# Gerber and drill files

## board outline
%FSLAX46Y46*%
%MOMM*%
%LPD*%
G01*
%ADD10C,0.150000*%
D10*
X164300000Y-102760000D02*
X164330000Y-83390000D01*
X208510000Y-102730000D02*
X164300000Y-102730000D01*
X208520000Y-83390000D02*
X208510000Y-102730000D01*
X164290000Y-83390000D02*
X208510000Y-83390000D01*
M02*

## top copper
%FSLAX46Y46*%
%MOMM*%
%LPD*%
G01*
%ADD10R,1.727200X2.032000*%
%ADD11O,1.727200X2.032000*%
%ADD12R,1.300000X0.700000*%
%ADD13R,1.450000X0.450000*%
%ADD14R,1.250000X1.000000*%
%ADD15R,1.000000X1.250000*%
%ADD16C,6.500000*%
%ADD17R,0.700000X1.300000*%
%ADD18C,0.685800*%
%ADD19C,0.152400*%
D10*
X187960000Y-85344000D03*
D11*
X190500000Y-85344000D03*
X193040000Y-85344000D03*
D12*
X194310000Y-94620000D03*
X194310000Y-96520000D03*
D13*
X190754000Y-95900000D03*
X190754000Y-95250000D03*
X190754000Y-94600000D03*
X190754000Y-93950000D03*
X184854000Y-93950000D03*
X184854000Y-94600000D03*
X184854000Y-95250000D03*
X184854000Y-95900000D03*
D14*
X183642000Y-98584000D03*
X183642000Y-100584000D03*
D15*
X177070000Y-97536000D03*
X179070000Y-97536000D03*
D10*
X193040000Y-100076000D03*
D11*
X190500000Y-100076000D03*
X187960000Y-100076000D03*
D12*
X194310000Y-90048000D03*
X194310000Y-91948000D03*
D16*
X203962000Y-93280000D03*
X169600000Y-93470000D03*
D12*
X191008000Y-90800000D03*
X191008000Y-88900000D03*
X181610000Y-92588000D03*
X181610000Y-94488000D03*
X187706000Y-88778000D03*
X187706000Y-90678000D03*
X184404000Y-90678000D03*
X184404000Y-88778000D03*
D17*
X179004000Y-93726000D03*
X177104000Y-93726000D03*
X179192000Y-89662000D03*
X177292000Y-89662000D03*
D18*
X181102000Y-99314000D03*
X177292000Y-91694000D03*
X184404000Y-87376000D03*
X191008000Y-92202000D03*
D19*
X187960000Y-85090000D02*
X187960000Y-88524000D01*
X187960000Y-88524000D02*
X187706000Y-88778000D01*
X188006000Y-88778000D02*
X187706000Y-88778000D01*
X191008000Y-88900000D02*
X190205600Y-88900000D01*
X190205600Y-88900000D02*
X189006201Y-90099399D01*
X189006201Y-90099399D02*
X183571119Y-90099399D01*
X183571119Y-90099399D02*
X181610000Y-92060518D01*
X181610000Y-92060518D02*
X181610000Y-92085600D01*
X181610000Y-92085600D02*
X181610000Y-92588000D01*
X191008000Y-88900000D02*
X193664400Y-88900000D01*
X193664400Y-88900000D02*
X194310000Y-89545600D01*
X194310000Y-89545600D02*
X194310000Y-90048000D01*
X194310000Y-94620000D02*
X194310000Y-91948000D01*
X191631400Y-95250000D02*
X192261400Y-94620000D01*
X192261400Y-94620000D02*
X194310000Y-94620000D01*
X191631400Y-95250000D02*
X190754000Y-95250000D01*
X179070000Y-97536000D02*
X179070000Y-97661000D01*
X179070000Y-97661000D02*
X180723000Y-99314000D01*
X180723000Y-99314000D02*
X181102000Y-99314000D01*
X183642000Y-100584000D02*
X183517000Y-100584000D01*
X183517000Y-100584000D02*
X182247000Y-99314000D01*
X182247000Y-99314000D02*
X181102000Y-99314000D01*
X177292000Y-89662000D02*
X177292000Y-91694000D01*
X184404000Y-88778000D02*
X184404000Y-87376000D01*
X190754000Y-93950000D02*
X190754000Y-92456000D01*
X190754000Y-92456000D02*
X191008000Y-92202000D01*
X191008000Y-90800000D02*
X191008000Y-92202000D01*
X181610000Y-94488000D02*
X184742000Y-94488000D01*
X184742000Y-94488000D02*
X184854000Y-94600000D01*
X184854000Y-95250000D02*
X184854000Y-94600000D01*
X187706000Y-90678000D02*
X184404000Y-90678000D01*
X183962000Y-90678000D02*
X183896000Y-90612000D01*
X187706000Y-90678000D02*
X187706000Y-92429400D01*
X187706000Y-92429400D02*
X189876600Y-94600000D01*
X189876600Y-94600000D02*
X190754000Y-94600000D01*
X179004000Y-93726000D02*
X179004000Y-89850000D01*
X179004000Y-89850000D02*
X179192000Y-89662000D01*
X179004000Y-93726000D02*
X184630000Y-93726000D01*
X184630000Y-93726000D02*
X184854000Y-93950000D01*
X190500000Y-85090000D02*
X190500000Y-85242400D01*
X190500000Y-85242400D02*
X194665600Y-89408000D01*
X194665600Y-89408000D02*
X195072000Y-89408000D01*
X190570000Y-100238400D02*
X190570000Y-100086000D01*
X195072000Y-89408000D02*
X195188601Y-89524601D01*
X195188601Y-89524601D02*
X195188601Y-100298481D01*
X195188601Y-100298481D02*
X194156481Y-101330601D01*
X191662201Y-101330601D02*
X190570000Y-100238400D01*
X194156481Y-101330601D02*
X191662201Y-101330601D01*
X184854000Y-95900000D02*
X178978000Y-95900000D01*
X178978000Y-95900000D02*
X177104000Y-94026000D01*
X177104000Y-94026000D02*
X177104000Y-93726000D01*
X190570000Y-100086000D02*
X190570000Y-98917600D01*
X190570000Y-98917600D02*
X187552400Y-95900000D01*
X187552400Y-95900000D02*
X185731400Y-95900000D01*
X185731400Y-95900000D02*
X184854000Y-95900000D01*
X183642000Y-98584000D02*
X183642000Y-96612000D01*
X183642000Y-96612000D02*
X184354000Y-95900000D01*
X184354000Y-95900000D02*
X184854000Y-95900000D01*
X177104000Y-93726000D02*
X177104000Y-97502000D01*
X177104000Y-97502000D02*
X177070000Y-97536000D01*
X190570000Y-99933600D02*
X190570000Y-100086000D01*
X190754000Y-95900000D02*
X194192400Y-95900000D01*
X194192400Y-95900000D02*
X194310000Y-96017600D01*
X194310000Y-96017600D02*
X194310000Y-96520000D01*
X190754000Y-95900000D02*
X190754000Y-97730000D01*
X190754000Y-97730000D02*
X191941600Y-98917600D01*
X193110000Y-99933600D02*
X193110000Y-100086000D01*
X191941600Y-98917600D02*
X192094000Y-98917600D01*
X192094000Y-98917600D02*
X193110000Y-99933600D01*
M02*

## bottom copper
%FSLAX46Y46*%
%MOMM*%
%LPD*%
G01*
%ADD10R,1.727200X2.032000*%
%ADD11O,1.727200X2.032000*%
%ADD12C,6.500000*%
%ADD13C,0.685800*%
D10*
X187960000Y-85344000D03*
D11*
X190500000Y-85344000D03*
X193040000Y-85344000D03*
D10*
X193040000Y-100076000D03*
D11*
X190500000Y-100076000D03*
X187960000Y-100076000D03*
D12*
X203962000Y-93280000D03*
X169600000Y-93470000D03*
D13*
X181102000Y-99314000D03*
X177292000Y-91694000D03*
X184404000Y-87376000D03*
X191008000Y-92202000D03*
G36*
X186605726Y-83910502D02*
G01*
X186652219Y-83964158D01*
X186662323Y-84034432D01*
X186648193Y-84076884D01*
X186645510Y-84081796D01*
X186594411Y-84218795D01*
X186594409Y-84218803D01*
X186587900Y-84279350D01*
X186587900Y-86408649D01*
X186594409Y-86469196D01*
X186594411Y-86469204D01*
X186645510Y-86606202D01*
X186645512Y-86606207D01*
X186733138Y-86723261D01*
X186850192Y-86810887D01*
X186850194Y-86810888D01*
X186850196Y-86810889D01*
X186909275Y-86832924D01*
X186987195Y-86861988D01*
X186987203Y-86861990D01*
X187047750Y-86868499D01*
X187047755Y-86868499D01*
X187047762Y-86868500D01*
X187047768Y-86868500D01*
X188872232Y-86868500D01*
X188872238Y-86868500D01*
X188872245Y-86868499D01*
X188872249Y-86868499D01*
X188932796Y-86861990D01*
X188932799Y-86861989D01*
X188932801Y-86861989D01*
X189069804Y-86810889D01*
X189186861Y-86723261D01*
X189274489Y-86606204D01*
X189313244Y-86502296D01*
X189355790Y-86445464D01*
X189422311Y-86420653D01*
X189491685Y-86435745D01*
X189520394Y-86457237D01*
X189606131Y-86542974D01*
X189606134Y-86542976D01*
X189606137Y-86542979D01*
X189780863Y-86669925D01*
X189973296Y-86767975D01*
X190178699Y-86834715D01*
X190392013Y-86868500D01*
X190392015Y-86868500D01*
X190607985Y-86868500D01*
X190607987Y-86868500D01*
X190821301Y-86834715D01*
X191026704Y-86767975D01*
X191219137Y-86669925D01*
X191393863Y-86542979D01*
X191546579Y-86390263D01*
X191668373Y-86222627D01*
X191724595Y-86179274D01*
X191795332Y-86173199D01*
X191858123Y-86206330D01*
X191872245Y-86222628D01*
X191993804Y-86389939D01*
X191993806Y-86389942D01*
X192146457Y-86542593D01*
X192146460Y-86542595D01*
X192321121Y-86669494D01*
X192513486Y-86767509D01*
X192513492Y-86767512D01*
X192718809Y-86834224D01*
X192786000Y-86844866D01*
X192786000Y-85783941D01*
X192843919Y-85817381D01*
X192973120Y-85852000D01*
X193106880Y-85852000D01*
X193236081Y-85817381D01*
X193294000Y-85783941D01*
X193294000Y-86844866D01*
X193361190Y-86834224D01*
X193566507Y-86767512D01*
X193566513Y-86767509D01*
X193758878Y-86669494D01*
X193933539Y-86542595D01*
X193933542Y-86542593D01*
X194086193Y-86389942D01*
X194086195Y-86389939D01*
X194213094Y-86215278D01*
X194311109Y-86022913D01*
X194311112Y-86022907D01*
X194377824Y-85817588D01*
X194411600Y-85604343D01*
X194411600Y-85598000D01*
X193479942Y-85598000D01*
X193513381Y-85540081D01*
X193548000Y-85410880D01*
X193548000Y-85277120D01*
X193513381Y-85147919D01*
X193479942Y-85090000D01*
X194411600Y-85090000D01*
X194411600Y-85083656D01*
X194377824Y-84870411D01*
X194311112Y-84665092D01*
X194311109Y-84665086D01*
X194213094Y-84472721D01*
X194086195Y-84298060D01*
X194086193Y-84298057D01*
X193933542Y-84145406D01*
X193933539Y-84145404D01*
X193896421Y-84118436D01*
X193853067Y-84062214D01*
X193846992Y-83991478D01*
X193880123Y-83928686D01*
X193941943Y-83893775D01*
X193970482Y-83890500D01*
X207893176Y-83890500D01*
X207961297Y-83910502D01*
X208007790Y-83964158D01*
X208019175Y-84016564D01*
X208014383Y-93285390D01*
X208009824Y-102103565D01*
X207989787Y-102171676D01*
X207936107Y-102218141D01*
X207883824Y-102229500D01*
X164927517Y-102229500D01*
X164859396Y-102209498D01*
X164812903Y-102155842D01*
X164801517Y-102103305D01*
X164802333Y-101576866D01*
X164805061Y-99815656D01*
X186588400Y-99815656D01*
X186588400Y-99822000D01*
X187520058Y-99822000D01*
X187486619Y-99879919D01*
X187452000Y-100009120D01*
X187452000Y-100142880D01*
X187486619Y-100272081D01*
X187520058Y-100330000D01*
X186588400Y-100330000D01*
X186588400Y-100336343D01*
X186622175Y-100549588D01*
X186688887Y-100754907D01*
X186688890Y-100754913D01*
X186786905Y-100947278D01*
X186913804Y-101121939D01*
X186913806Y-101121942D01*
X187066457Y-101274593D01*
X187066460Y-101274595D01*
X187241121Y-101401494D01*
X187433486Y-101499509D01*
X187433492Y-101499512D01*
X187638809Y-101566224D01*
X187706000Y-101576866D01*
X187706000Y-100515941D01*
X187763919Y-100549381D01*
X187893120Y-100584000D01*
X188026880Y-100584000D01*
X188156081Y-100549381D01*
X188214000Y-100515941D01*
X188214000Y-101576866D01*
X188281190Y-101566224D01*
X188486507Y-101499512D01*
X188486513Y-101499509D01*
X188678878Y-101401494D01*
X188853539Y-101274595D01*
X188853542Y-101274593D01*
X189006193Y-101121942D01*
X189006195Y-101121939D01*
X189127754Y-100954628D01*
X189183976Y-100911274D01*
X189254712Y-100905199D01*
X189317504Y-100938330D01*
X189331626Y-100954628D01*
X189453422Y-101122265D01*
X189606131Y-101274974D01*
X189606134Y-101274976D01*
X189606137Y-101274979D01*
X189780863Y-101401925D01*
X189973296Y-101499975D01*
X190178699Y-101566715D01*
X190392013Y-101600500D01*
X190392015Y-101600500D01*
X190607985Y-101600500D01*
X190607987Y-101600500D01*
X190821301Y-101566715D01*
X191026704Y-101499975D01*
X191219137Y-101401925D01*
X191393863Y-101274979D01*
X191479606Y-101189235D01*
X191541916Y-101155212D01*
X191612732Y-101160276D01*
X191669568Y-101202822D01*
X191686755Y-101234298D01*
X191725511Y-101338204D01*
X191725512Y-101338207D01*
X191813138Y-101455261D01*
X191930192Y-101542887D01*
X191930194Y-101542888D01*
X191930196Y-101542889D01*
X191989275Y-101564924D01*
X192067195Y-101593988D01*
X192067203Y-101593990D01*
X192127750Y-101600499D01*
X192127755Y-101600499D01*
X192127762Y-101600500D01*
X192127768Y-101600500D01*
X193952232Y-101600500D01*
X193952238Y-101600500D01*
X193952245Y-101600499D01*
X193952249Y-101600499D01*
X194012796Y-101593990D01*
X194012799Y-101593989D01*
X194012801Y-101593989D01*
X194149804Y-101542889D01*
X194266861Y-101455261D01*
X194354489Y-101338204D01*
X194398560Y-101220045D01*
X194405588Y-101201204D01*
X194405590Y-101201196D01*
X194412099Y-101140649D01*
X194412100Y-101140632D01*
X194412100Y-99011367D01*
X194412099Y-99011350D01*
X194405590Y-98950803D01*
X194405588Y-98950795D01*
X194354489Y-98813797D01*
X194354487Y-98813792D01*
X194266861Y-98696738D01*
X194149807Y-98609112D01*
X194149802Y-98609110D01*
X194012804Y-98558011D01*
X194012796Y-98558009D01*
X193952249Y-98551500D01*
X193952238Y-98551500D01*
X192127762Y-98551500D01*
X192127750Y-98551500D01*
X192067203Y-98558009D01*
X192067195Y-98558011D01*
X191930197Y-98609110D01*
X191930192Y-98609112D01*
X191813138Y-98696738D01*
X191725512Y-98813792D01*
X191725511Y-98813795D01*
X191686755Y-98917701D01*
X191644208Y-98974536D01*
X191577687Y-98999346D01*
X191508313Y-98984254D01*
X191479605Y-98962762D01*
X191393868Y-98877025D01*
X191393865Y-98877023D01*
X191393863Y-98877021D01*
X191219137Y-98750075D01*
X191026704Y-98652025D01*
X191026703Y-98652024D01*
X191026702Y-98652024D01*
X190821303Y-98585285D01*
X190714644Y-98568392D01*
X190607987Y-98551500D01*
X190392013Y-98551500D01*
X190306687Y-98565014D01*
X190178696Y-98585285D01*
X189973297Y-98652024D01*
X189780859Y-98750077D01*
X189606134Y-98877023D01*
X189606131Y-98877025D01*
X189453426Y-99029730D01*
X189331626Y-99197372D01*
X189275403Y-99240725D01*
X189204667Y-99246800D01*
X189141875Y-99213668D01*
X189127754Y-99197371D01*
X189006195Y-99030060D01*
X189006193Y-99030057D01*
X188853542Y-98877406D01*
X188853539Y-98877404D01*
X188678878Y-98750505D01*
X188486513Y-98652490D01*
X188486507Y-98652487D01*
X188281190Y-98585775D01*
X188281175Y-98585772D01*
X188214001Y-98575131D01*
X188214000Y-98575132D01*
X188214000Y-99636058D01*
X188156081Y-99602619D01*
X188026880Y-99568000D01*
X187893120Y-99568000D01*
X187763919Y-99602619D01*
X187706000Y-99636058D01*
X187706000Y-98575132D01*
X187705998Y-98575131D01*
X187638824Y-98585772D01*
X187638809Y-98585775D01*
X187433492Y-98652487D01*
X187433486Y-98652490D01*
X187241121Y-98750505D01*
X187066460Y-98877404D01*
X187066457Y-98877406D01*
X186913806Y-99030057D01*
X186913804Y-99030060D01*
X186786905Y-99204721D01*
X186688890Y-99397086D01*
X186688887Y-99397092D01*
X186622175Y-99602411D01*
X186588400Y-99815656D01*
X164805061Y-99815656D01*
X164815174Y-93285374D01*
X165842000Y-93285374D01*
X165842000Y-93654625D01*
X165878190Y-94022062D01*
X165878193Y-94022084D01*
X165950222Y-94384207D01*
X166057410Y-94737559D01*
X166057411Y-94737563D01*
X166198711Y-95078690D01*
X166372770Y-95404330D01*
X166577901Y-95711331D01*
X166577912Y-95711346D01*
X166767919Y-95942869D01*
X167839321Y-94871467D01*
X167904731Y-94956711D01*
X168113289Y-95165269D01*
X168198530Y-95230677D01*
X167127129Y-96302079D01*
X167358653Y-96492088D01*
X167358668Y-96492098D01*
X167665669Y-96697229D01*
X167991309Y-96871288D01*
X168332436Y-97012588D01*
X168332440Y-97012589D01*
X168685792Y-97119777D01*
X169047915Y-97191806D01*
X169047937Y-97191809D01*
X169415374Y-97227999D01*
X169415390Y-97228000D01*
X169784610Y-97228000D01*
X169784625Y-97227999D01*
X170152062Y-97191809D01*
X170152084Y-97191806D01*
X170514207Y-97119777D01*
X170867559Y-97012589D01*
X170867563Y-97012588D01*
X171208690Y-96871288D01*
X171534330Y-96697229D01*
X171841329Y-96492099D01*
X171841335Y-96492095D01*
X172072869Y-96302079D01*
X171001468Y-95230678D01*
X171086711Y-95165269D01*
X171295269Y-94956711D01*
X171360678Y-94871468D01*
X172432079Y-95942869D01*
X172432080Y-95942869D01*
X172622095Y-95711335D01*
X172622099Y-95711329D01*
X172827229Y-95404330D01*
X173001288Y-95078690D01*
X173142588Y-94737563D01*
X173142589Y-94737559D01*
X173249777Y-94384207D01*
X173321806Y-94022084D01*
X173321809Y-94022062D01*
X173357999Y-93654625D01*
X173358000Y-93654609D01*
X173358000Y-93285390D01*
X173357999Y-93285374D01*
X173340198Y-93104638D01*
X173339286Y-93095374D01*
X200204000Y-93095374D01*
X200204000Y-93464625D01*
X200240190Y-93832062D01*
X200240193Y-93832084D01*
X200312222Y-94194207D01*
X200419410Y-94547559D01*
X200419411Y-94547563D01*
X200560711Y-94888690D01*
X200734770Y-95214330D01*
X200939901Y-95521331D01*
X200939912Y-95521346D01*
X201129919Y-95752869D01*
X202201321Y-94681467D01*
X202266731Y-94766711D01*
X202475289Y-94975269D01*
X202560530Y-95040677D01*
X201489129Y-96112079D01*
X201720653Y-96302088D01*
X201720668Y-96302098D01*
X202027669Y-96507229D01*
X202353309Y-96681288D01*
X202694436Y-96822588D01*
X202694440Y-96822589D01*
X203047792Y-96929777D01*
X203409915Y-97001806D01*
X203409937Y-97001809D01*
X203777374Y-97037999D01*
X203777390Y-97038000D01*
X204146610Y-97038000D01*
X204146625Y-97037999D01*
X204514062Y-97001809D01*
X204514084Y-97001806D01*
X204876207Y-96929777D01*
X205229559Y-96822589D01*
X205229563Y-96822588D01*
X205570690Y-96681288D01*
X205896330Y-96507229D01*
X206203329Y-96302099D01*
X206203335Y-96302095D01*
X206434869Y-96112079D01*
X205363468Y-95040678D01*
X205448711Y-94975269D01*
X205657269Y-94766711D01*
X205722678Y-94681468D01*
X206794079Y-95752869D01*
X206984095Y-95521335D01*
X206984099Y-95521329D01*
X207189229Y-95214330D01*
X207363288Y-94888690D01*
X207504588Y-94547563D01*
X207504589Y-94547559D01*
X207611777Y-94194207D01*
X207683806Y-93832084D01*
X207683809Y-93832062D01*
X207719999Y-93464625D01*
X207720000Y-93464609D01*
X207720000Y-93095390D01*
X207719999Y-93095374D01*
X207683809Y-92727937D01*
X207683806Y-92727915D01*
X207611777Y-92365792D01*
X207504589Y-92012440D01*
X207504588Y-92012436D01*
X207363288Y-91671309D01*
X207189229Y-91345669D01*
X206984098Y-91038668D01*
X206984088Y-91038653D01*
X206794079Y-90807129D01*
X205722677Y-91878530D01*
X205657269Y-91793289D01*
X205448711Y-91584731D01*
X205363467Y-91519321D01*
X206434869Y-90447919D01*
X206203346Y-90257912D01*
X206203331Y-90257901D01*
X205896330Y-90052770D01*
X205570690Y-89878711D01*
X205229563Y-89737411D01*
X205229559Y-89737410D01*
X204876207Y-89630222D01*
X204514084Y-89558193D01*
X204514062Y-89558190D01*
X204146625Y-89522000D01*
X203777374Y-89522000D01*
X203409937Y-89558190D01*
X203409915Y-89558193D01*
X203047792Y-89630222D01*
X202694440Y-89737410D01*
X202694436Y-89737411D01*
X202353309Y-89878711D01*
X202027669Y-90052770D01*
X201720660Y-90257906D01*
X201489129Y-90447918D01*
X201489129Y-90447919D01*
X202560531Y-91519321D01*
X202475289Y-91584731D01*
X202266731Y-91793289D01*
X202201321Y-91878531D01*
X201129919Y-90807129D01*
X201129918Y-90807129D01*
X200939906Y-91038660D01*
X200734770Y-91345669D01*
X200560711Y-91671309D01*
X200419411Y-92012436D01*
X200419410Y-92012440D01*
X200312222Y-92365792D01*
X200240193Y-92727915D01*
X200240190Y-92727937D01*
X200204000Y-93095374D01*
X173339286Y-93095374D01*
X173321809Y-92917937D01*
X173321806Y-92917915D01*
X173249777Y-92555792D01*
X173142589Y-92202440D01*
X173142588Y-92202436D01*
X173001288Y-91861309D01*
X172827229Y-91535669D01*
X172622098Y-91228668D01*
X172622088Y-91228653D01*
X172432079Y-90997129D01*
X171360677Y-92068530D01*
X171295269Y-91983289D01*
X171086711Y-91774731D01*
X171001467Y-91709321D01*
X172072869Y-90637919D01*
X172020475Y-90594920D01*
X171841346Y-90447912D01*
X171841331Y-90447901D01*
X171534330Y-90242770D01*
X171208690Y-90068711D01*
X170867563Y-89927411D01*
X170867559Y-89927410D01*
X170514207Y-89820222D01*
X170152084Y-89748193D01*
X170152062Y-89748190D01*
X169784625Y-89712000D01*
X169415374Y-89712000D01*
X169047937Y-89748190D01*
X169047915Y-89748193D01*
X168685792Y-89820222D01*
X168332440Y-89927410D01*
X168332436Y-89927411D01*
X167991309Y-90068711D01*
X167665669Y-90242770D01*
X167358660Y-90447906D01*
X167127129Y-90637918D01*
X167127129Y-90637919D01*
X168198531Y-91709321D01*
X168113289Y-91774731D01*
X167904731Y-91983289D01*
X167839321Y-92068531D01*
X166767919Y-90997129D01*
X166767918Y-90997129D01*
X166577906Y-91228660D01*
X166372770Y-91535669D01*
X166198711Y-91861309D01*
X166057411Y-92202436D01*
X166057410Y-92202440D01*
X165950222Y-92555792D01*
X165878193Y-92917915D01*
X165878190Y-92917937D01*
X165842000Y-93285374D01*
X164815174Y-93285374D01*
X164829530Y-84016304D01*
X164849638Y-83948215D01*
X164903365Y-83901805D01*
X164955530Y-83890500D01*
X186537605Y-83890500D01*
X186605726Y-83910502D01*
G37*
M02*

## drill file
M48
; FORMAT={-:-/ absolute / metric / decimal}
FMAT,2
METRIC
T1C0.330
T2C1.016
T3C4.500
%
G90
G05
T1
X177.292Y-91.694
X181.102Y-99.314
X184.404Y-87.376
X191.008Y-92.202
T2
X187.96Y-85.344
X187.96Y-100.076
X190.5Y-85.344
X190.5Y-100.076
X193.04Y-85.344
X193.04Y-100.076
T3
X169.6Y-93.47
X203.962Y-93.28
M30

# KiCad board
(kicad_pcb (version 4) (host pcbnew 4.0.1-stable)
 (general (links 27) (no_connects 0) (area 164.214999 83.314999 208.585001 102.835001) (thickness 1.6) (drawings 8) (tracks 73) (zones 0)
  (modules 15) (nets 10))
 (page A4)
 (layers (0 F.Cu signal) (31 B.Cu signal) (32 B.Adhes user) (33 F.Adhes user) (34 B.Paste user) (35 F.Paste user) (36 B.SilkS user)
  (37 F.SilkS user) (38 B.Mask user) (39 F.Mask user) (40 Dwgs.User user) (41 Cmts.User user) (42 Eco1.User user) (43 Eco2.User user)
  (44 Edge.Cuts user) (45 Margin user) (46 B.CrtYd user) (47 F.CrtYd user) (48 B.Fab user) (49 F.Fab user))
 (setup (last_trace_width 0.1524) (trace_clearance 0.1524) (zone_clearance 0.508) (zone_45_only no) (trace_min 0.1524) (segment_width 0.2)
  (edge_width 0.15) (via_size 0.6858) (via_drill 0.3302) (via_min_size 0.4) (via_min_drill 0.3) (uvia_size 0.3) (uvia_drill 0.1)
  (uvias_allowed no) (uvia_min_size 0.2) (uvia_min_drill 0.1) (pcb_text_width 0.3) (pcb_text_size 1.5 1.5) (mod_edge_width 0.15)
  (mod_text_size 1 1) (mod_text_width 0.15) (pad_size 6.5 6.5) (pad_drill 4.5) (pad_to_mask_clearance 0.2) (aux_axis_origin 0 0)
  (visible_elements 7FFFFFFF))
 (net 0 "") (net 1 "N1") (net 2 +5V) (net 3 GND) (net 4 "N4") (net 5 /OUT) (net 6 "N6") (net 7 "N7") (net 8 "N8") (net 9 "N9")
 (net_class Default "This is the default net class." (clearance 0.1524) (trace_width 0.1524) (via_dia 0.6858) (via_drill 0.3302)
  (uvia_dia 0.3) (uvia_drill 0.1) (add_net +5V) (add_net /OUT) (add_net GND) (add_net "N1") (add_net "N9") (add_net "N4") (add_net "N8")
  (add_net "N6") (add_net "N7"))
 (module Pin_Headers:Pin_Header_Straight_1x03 (layer F.Cu) (at 187.96 85.344 90)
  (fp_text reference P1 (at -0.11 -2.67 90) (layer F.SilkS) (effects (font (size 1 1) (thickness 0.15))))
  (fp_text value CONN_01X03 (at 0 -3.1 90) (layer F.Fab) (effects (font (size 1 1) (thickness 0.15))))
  (pad 1 thru_hole rect (at 0 0 90) (size 2.032 1.7272) (drill 1.016) (layers *.Cu *.Mask F.SilkS) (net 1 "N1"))
  (pad 2 thru_hole oval (at 0 2.54 90) (size 2.032 1.7272) (drill 1.016) (layers *.Cu *.Mask F.SilkS) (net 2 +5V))
  (pad 3 thru_hole oval (at 0 5.08 90) (size 2.032 1.7272) (drill 1.016) (layers *.Cu *.Mask F.SilkS) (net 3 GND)))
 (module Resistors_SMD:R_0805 (layer F.Cu) (at 194.31 95.57 270)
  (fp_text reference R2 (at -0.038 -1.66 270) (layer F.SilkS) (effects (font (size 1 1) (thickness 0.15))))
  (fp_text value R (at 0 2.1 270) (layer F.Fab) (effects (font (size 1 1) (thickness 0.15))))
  (pad 1 smd rect (at -0.95 0 270) (size 0.7 1.3) (layers F.Cu F.Paste F.Mask) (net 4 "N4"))
  (pad 2 smd rect (at 0.95 0 270) (size 0.7 1.3) (layers F.Cu F.Paste F.Mask) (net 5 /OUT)))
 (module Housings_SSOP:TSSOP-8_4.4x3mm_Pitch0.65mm (layer F.Cu) (at 187.804 94.925 180)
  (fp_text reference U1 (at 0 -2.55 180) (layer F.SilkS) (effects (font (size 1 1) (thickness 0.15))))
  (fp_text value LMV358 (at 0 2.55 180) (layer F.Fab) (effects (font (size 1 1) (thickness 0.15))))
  (pad 1 smd rect (at -2.95 -0.975 180) (size 1.45 0.45) (layers F.Cu F.Paste F.Mask) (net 5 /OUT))
  (pad 2 smd rect (at -2.95 -0.325 180) (size 1.45 0.45) (layers F.Cu F.Paste F.Mask) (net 4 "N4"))
  (pad 3 smd rect (at -2.95 0.325 180) (size 1.45 0.45) (layers F.Cu F.Paste F.Mask) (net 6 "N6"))
  (pad 4 smd rect (at -2.95 0.975 180) (size 1.45 0.45) (layers F.Cu F.Paste F.Mask) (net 3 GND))
  (pad 5 smd rect (at 2.95 0.975 180) (size 1.45 0.45) (layers F.Cu F.Paste F.Mask) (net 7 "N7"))
  (pad 6 smd rect (at 2.95 0.325 180) (size 1.45 0.45) (layers F.Cu F.Paste F.Mask) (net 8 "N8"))
  (pad 7 smd rect (at 2.95 -0.325 180) (size 1.45 0.45) (layers F.Cu F.Paste F.Mask) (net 8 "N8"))
  (pad 8 smd rect (at 2.95 -0.975 180) (size 1.45 0.45) (layers F.Cu F.Paste F.Mask) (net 2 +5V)))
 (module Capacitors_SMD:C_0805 (layer F.Cu) (at 183.642 99.584 270)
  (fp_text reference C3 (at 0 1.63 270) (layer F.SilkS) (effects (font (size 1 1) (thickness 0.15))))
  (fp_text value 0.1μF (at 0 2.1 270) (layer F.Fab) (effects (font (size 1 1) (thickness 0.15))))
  (pad 1 smd rect (at -1 0 270) (size 1 1.25) (layers F.Cu F.Paste F.Mask) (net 2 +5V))
  (pad 2 smd rect (at 1 0 270) (size 1 1.25) (layers F.Cu F.Paste F.Mask) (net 3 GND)))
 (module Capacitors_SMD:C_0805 (layer F.Cu) (at 178.07 97.536)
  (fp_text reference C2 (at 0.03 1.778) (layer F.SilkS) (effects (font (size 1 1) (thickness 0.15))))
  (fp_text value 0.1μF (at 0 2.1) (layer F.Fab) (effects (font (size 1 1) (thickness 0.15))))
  (pad 1 smd rect (at -1 0) (size 1 1.25) (layers F.Cu F.Paste F.Mask) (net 2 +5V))
  (pad 2 smd rect (at 1 0) (size 1 1.25) (layers F.Cu F.Paste F.Mask) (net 3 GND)))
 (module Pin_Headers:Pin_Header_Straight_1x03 (layer F.Cu) (at 193.04 100.076 270)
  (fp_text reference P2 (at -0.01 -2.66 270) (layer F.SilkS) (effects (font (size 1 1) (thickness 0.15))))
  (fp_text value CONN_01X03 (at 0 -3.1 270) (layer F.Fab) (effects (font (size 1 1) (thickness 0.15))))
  (pad 1 thru_hole rect (at 0 0 270) (size 2.032 1.7272) (drill 1.016) (layers *.Cu *.Mask F.SilkS) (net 5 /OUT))
  (pad 2 thru_hole oval (at 0 2.54 270) (size 2.032 1.7272) (drill 1.016) (layers *.Cu *.Mask F.SilkS) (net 2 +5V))
  (pad 3 thru_hole oval (at 0 5.08 270) (size 2.032 1.7272) (drill 1.016) (layers *.Cu *.Mask F.SilkS) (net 3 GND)))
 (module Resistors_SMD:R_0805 (layer F.Cu) (at 194.31 90.998 270)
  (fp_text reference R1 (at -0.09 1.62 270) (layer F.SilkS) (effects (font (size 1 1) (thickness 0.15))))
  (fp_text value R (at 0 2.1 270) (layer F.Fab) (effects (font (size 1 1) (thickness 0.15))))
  (pad 1 smd rect (at -0.95 0 270) (size 0.7 1.3) (layers F.Cu F.Paste F.Mask) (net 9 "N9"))
  (pad 2 smd rect (at 0.95 0 270) (size 0.7 1.3) (layers F.Cu F.Paste F.Mask) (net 4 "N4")))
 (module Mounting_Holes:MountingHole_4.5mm (layer F.Cu) (at 203.962 93.28)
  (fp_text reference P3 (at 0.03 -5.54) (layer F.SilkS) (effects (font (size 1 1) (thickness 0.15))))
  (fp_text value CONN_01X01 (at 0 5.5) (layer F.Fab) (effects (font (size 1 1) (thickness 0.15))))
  (pad 1 thru_hole circle (at 0 0) (size 6.5 6.5) (drill 4.5) (layers *.Cu *.Mask F.SilkS) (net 3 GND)))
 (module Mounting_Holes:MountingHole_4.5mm (layer F.Cu) (at 169.6 93.47)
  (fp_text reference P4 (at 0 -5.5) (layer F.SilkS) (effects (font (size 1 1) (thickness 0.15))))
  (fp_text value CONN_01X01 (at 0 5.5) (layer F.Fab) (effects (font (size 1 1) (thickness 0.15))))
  (pad 1 thru_hole circle (at 0 0) (size 6.5 6.5) (drill 4.5) (layers *.Cu *.Mask F.SilkS) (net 3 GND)))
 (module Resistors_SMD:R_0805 (layer F.Cu) (at 191.008 89.85 90)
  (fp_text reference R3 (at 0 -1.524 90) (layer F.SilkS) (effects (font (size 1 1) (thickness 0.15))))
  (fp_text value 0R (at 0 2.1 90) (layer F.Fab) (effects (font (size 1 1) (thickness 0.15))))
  (pad 1 smd rect (at -0.95 0 90) (size 0.7 1.3) (layers F.Cu F.Paste F.Mask) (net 3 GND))
  (pad 2 smd rect (at 0.95 0 90) (size 0.7 1.3) (layers F.Cu F.Paste F.Mask) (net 9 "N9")))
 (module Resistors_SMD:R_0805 (layer F.Cu) (at 181.61 93.538 270)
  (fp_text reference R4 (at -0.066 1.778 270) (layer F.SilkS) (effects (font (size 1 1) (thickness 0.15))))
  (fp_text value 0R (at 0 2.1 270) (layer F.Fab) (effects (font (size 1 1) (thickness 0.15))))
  (pad 1 smd rect (at -0.95 0 270) (size 0.7 1.3) (layers F.Cu F.Paste F.Mask) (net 9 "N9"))
  (pad 2 smd rect (at 0.95 0 270) (size 0.7 1.3) (layers F.Cu F.Paste F.Mask) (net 8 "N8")))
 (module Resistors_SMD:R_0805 (layer F.Cu) (at 187.706 89.728 270)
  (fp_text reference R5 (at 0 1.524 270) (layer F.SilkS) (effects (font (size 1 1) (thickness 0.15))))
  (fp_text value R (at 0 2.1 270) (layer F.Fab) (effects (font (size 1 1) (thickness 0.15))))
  (pad 1 smd rect (at -0.95 0 270) (size 0.7 1.3) (layers F.Cu F.Paste F.Mask) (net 1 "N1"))
  (pad 2 smd rect (at 0.95 0 270) (size 0.7 1.3) (layers F.Cu F.Paste F.Mask) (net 6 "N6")))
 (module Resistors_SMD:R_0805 (layer F.Cu) (at 184.404 89.728 90)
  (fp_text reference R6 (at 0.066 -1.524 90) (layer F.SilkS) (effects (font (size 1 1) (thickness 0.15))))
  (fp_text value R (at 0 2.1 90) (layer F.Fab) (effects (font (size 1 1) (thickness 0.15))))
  (pad 1 smd rect (at -0.95 0 90) (size 0.7 1.3) (layers F.Cu F.Paste F.Mask) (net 6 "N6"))
  (pad 2 smd rect (at 0.95 0 90) (size 0.7 1.3) (layers F.Cu F.Paste F.Mask) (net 3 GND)))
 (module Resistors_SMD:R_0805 (layer F.Cu) (at 178.054 93.726 180)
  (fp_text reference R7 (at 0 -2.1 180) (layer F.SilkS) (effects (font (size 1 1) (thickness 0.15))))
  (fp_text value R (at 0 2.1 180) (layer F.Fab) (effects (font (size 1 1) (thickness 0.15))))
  (pad 1 smd rect (at -0.95 0 180) (size 0.7 1.3) (layers F.Cu F.Paste F.Mask) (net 7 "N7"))
  (pad 2 smd rect (at 0.95 0 180) (size 0.7 1.3) (layers F.Cu F.Paste F.Mask) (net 2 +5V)))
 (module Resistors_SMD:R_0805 (layer F.Cu) (at 178.242 89.662 180)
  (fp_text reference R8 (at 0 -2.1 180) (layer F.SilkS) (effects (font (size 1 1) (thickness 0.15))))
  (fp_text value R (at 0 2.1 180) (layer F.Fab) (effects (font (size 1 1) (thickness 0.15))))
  (pad 1 smd rect (at -0.95 0 180) (size 0.7 1.3) (layers F.Cu F.Paste F.Mask) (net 7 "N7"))
  (pad 2 smd rect (at 0.95 0 180) (size 0.7 1.3) (layers F.Cu F.Paste F.Mask) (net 3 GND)))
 (gr_line (start 164.3 102.76) (end 164.33 83.39) (angle 90) (layer Edge.Cuts) (width 0.15))
 (gr_line (start 208.51 102.73) (end 164.3 102.73) (angle 90) (layer Edge.Cuts) (width 0.15))
 (gr_line (start 208.52 83.39) (end 208.51 102.73) (angle 90) (layer Edge.Cuts) (width 0.15))
 (gr_line (start 164.29 83.39) (end 208.51 83.39) (angle 90) (layer Edge.Cuts) (width 0.15))
 (segment (start 187.96 85.09) (end 187.96 88.524) (width 0.1524) (layer F.Cu) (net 1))
 (segment (start 187.96 88.524) (end 187.706 88.778) (width 0.1524) (layer F.Cu) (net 1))
 (segment (start 188.006 88.778) (end 187.706 88.778) (width 0.1524) (layer F.Cu) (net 1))
 (segment (start 191.008 88.9) (end 190.2056 88.9) (width 0.1524) (layer F.Cu) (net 9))
 (segment (start 190.2056 88.9) (end 189.006201 90.099399) (width 0.1524) (layer F.Cu) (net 9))
 (segment (start 189.006201 90.099399) (end 183.571119 90.099399) (width 0.1524) (layer F.Cu) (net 9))
 (segment (start 183.571119 90.099399) (end 181.61 92.060518) (width 0.1524) (layer F.Cu) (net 9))
 (segment (start 181.61 92.060518) (end 181.61 92.0856) (width 0.1524) (layer F.Cu) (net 9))
 (segment (start 181.61 92.0856) (end 181.61 92.588) (width 0.1524) (layer F.Cu) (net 9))
 (segment (start 191.008 88.9) (end 193.6644 88.9) (width 0.1524) (layer F.Cu) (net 9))
 (segment (start 193.6644 88.9) (end 194.31 89.5456) (width 0.1524) (layer F.Cu) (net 9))
 (segment (start 194.31 89.5456) (end 194.31 90.048) (width 0.1524) (layer F.Cu) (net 9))
 (segment (start 194.31 94.62) (end 194.31 91.948) (width 0.1524) (layer F.Cu) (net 4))
 (segment (start 191.6314 95.25) (end 192.2614 94.62) (width 0.1524) (layer F.Cu) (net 4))
 (segment (start 192.2614 94.62) (end 194.31 94.62) (width 0.1524) (layer F.Cu) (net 4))
 (segment (start 191.6314 95.25) (end 190.754 95.25) (width 0.1524) (layer F.Cu) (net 4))
 (segment (start 179.07 97.536) (end 179.07 97.661) (width 0.1524) (layer F.Cu) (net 3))
 (segment (start 179.07 97.661) (end 180.723 99.314) (width 0.1524) (layer F.Cu) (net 3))
 (segment (start 180.723 99.314) (end 181.102 99.314) (width 0.1524) (layer F.Cu) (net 3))
 (segment (start 183.642 100.584) (end 183.517 100.584) (width 0.1524) (layer F.Cu) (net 3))
 (segment (start 183.517 100.584) (end 182.247 99.314) (width 0.1524) (layer F.Cu) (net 3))
 (segment (start 182.247 99.314) (end 181.102 99.314) (width 0.1524) (layer F.Cu) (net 3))
 (via (at 181.102 99.314) (size 0.6858) (drill 0.3302) (layers F.Cu B.Cu) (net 3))
 (segment (start 177.292 89.662) (end 177.292 91.694) (width 0.1524) (layer F.Cu) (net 3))
 (via (at 177.292 91.694) (size 0.6858) (drill 0.3302) (layers F.Cu B.Cu) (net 3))
 (segment (start 184.404 88.778) (end 184.404 87.376) (width 0.1524) (layer F.Cu) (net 3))
 (via (at 184.404 87.376) (size 0.6858) (drill 0.3302) (layers F.Cu B.Cu) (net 3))
 (segment (start 190.754 93.95) (end 190.754 92.456) (width 0.1524) (layer F.Cu) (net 3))
 (segment (start 190.754 92.456) (end 191.008 92.202) (width 0.1524) (layer F.Cu) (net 3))
 (segment (start 191.008 90.8) (end 191.008 92.202) (width 0.1524) (layer F.Cu) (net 3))
 (via (at 191.008 92.202) (size 0.6858) (drill 0.3302) (layers F.Cu B.Cu) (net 3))
 (segment (start 181.61 94.488) (end 184.742 94.488) (width 0.1524) (layer F.Cu) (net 8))
 (segment (start 184.742 94.488) (end 184.854 94.6) (width 0.1524) (layer F.Cu) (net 8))
 (segment (start 184.854 95.25) (end 184.854 94.6) (width 0.1524) (layer F.Cu) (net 8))
 (segment (start 187.706 90.678) (end 184.404 90.678) (width 0.1524) (layer F.Cu) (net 6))
 (segment (start 183.962 90.678) (end 183.896 90.612) (width 0.1524) (layer F.Cu) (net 6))
 (segment (start 187.706 90.678) (end 187.706 92.4294) (width 0.1524) (layer F.Cu) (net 6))
 (segment (start 187.706 92.4294) (end 189.8766 94.6) (width 0.1524) (layer F.Cu) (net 6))
 (segment (start 189.8766 94.6) (end 190.754 94.6) (width 0.1524) (layer F.Cu) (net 6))
 (segment (start 179.004 93.726) (end 179.004 89.85) (width 0.1524) (layer F.Cu) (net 7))
 (segment (start 179.004 89.85) (end 179.192 89.662) (width 0.1524) (layer F.Cu) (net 7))
 (segment (start 179.004 93.726) (end 184.63 93.726) (width 0.1524) (layer F.Cu) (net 7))
 (segment (start 184.63 93.726) (end 184.854 93.95) (width 0.1524) (layer F.Cu) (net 7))
 (segment (start 190.5 85.09) (end 190.5 85.2424) (width 0.1524) (layer F.Cu) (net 2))
 (segment (start 190.5 85.2424) (end 194.6656 89.408) (width 0.1524) (layer F.Cu) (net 2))
 (segment (start 194.6656 89.408) (end 195.072 89.408) (width 0.1524) (layer F.Cu) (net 2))
 (segment (start 190.57 100.2384) (end 190.57 100.086) (width 0.1524) (layer F.Cu) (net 2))
 (segment (start 195.072 89.408) (end 195.188601 89.524601) (width 0.1524) (layer F.Cu) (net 2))
 (segment (start 195.188601 89.524601) (end 195.188601 100.298481) (width 0.1524) (layer F.Cu) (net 2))
 (segment (start 195.188601 100.298481) (end 194.156481 101.330601) (width 0.1524) (layer F.Cu) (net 2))
 (segment (start 191.662201 101.330601) (end 190.57 100.2384) (width 0.1524) (layer F.Cu) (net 2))
 (segment (start 194.156481 101.330601) (end 191.662201 101.330601) (width 0.1524) (layer F.Cu) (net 2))
 (segment (start 184.854 95.9) (end 178.978 95.9) (width 0.1524) (layer F.Cu) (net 2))
 (segment (start 178.978 95.9) (end 177.104 94.026) (width 0.1524) (layer F.Cu) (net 2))
 (segment (start 177.104 94.026) (end 177.104 93.726) (width 0.1524) (layer F.Cu) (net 2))
 (segment (start 190.57 100.086) (end 190.57 98.9176) (width 0.1524) (layer F.Cu) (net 2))
 (segment (start 190.57 98.9176) (end 187.5524 95.9) (width 0.1524) (layer F.Cu) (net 2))
 (segment (start 187.5524 95.9) (end 185.7314 95.9) (width 0.1524) (layer F.Cu) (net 2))
 (segment (start 185.7314 95.9) (end 184.854 95.9) (width 0.1524) (layer F.Cu) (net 2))
 (segment (start 183.642 98.584) (end 183.642 96.612) (width 0.1524) (layer F.Cu) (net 2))
 (segment (start 183.642 96.612) (end 184.354 95.9) (width 0.1524) (layer F.Cu) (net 2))
 (segment (start 184.354 95.9) (end 184.854 95.9) (width 0.1524) (layer F.Cu) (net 2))
 (segment (start 177.104 93.726) (end 177.104 97.502) (width 0.1524) (layer F.Cu) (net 2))
 (segment (start 177.104 97.502) (end 177.07 97.536) (width 0.1524) (layer F.Cu) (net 2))
 (segment (start 190.57 99.9336) (end 190.57 100.086) (width 0.1524) (layer F.Cu) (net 2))
 (segment (start 190.754 95.9) (end 194.1924 95.9) (width 0.1524) (layer F.Cu) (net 5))
 (segment (start 194.1924 95.9) (end 194.31 96.0176) (width 0.1524) (layer F.Cu) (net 5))
 (segment (start 194.31 96.0176) (end 194.31 96.52) (width 0.1524) (layer F.Cu) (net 5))
 (segment (start 190.754 95.9) (end 190.754 97.73) (width 0.1524) (layer F.Cu) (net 5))
 (segment (start 190.754 97.73) (end 191.9416 98.9176) (width 0.1524) (layer F.Cu) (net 5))
 (segment (start 193.11 99.9336) (end 193.11 100.086) (width 0.1524) (layer F.Cu) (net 5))
 (segment (start 191.9416 98.9176) (end 192.094 98.9176) (width 0.1524) (layer F.Cu) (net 5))
 (segment (start 192.094 98.9176) (end 193.11 99.9336) (width 0.1524) (layer F.Cu) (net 5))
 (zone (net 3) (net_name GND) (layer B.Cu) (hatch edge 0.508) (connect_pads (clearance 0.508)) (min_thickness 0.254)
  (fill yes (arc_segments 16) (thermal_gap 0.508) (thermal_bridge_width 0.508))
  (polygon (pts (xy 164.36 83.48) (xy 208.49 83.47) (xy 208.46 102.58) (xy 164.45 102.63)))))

